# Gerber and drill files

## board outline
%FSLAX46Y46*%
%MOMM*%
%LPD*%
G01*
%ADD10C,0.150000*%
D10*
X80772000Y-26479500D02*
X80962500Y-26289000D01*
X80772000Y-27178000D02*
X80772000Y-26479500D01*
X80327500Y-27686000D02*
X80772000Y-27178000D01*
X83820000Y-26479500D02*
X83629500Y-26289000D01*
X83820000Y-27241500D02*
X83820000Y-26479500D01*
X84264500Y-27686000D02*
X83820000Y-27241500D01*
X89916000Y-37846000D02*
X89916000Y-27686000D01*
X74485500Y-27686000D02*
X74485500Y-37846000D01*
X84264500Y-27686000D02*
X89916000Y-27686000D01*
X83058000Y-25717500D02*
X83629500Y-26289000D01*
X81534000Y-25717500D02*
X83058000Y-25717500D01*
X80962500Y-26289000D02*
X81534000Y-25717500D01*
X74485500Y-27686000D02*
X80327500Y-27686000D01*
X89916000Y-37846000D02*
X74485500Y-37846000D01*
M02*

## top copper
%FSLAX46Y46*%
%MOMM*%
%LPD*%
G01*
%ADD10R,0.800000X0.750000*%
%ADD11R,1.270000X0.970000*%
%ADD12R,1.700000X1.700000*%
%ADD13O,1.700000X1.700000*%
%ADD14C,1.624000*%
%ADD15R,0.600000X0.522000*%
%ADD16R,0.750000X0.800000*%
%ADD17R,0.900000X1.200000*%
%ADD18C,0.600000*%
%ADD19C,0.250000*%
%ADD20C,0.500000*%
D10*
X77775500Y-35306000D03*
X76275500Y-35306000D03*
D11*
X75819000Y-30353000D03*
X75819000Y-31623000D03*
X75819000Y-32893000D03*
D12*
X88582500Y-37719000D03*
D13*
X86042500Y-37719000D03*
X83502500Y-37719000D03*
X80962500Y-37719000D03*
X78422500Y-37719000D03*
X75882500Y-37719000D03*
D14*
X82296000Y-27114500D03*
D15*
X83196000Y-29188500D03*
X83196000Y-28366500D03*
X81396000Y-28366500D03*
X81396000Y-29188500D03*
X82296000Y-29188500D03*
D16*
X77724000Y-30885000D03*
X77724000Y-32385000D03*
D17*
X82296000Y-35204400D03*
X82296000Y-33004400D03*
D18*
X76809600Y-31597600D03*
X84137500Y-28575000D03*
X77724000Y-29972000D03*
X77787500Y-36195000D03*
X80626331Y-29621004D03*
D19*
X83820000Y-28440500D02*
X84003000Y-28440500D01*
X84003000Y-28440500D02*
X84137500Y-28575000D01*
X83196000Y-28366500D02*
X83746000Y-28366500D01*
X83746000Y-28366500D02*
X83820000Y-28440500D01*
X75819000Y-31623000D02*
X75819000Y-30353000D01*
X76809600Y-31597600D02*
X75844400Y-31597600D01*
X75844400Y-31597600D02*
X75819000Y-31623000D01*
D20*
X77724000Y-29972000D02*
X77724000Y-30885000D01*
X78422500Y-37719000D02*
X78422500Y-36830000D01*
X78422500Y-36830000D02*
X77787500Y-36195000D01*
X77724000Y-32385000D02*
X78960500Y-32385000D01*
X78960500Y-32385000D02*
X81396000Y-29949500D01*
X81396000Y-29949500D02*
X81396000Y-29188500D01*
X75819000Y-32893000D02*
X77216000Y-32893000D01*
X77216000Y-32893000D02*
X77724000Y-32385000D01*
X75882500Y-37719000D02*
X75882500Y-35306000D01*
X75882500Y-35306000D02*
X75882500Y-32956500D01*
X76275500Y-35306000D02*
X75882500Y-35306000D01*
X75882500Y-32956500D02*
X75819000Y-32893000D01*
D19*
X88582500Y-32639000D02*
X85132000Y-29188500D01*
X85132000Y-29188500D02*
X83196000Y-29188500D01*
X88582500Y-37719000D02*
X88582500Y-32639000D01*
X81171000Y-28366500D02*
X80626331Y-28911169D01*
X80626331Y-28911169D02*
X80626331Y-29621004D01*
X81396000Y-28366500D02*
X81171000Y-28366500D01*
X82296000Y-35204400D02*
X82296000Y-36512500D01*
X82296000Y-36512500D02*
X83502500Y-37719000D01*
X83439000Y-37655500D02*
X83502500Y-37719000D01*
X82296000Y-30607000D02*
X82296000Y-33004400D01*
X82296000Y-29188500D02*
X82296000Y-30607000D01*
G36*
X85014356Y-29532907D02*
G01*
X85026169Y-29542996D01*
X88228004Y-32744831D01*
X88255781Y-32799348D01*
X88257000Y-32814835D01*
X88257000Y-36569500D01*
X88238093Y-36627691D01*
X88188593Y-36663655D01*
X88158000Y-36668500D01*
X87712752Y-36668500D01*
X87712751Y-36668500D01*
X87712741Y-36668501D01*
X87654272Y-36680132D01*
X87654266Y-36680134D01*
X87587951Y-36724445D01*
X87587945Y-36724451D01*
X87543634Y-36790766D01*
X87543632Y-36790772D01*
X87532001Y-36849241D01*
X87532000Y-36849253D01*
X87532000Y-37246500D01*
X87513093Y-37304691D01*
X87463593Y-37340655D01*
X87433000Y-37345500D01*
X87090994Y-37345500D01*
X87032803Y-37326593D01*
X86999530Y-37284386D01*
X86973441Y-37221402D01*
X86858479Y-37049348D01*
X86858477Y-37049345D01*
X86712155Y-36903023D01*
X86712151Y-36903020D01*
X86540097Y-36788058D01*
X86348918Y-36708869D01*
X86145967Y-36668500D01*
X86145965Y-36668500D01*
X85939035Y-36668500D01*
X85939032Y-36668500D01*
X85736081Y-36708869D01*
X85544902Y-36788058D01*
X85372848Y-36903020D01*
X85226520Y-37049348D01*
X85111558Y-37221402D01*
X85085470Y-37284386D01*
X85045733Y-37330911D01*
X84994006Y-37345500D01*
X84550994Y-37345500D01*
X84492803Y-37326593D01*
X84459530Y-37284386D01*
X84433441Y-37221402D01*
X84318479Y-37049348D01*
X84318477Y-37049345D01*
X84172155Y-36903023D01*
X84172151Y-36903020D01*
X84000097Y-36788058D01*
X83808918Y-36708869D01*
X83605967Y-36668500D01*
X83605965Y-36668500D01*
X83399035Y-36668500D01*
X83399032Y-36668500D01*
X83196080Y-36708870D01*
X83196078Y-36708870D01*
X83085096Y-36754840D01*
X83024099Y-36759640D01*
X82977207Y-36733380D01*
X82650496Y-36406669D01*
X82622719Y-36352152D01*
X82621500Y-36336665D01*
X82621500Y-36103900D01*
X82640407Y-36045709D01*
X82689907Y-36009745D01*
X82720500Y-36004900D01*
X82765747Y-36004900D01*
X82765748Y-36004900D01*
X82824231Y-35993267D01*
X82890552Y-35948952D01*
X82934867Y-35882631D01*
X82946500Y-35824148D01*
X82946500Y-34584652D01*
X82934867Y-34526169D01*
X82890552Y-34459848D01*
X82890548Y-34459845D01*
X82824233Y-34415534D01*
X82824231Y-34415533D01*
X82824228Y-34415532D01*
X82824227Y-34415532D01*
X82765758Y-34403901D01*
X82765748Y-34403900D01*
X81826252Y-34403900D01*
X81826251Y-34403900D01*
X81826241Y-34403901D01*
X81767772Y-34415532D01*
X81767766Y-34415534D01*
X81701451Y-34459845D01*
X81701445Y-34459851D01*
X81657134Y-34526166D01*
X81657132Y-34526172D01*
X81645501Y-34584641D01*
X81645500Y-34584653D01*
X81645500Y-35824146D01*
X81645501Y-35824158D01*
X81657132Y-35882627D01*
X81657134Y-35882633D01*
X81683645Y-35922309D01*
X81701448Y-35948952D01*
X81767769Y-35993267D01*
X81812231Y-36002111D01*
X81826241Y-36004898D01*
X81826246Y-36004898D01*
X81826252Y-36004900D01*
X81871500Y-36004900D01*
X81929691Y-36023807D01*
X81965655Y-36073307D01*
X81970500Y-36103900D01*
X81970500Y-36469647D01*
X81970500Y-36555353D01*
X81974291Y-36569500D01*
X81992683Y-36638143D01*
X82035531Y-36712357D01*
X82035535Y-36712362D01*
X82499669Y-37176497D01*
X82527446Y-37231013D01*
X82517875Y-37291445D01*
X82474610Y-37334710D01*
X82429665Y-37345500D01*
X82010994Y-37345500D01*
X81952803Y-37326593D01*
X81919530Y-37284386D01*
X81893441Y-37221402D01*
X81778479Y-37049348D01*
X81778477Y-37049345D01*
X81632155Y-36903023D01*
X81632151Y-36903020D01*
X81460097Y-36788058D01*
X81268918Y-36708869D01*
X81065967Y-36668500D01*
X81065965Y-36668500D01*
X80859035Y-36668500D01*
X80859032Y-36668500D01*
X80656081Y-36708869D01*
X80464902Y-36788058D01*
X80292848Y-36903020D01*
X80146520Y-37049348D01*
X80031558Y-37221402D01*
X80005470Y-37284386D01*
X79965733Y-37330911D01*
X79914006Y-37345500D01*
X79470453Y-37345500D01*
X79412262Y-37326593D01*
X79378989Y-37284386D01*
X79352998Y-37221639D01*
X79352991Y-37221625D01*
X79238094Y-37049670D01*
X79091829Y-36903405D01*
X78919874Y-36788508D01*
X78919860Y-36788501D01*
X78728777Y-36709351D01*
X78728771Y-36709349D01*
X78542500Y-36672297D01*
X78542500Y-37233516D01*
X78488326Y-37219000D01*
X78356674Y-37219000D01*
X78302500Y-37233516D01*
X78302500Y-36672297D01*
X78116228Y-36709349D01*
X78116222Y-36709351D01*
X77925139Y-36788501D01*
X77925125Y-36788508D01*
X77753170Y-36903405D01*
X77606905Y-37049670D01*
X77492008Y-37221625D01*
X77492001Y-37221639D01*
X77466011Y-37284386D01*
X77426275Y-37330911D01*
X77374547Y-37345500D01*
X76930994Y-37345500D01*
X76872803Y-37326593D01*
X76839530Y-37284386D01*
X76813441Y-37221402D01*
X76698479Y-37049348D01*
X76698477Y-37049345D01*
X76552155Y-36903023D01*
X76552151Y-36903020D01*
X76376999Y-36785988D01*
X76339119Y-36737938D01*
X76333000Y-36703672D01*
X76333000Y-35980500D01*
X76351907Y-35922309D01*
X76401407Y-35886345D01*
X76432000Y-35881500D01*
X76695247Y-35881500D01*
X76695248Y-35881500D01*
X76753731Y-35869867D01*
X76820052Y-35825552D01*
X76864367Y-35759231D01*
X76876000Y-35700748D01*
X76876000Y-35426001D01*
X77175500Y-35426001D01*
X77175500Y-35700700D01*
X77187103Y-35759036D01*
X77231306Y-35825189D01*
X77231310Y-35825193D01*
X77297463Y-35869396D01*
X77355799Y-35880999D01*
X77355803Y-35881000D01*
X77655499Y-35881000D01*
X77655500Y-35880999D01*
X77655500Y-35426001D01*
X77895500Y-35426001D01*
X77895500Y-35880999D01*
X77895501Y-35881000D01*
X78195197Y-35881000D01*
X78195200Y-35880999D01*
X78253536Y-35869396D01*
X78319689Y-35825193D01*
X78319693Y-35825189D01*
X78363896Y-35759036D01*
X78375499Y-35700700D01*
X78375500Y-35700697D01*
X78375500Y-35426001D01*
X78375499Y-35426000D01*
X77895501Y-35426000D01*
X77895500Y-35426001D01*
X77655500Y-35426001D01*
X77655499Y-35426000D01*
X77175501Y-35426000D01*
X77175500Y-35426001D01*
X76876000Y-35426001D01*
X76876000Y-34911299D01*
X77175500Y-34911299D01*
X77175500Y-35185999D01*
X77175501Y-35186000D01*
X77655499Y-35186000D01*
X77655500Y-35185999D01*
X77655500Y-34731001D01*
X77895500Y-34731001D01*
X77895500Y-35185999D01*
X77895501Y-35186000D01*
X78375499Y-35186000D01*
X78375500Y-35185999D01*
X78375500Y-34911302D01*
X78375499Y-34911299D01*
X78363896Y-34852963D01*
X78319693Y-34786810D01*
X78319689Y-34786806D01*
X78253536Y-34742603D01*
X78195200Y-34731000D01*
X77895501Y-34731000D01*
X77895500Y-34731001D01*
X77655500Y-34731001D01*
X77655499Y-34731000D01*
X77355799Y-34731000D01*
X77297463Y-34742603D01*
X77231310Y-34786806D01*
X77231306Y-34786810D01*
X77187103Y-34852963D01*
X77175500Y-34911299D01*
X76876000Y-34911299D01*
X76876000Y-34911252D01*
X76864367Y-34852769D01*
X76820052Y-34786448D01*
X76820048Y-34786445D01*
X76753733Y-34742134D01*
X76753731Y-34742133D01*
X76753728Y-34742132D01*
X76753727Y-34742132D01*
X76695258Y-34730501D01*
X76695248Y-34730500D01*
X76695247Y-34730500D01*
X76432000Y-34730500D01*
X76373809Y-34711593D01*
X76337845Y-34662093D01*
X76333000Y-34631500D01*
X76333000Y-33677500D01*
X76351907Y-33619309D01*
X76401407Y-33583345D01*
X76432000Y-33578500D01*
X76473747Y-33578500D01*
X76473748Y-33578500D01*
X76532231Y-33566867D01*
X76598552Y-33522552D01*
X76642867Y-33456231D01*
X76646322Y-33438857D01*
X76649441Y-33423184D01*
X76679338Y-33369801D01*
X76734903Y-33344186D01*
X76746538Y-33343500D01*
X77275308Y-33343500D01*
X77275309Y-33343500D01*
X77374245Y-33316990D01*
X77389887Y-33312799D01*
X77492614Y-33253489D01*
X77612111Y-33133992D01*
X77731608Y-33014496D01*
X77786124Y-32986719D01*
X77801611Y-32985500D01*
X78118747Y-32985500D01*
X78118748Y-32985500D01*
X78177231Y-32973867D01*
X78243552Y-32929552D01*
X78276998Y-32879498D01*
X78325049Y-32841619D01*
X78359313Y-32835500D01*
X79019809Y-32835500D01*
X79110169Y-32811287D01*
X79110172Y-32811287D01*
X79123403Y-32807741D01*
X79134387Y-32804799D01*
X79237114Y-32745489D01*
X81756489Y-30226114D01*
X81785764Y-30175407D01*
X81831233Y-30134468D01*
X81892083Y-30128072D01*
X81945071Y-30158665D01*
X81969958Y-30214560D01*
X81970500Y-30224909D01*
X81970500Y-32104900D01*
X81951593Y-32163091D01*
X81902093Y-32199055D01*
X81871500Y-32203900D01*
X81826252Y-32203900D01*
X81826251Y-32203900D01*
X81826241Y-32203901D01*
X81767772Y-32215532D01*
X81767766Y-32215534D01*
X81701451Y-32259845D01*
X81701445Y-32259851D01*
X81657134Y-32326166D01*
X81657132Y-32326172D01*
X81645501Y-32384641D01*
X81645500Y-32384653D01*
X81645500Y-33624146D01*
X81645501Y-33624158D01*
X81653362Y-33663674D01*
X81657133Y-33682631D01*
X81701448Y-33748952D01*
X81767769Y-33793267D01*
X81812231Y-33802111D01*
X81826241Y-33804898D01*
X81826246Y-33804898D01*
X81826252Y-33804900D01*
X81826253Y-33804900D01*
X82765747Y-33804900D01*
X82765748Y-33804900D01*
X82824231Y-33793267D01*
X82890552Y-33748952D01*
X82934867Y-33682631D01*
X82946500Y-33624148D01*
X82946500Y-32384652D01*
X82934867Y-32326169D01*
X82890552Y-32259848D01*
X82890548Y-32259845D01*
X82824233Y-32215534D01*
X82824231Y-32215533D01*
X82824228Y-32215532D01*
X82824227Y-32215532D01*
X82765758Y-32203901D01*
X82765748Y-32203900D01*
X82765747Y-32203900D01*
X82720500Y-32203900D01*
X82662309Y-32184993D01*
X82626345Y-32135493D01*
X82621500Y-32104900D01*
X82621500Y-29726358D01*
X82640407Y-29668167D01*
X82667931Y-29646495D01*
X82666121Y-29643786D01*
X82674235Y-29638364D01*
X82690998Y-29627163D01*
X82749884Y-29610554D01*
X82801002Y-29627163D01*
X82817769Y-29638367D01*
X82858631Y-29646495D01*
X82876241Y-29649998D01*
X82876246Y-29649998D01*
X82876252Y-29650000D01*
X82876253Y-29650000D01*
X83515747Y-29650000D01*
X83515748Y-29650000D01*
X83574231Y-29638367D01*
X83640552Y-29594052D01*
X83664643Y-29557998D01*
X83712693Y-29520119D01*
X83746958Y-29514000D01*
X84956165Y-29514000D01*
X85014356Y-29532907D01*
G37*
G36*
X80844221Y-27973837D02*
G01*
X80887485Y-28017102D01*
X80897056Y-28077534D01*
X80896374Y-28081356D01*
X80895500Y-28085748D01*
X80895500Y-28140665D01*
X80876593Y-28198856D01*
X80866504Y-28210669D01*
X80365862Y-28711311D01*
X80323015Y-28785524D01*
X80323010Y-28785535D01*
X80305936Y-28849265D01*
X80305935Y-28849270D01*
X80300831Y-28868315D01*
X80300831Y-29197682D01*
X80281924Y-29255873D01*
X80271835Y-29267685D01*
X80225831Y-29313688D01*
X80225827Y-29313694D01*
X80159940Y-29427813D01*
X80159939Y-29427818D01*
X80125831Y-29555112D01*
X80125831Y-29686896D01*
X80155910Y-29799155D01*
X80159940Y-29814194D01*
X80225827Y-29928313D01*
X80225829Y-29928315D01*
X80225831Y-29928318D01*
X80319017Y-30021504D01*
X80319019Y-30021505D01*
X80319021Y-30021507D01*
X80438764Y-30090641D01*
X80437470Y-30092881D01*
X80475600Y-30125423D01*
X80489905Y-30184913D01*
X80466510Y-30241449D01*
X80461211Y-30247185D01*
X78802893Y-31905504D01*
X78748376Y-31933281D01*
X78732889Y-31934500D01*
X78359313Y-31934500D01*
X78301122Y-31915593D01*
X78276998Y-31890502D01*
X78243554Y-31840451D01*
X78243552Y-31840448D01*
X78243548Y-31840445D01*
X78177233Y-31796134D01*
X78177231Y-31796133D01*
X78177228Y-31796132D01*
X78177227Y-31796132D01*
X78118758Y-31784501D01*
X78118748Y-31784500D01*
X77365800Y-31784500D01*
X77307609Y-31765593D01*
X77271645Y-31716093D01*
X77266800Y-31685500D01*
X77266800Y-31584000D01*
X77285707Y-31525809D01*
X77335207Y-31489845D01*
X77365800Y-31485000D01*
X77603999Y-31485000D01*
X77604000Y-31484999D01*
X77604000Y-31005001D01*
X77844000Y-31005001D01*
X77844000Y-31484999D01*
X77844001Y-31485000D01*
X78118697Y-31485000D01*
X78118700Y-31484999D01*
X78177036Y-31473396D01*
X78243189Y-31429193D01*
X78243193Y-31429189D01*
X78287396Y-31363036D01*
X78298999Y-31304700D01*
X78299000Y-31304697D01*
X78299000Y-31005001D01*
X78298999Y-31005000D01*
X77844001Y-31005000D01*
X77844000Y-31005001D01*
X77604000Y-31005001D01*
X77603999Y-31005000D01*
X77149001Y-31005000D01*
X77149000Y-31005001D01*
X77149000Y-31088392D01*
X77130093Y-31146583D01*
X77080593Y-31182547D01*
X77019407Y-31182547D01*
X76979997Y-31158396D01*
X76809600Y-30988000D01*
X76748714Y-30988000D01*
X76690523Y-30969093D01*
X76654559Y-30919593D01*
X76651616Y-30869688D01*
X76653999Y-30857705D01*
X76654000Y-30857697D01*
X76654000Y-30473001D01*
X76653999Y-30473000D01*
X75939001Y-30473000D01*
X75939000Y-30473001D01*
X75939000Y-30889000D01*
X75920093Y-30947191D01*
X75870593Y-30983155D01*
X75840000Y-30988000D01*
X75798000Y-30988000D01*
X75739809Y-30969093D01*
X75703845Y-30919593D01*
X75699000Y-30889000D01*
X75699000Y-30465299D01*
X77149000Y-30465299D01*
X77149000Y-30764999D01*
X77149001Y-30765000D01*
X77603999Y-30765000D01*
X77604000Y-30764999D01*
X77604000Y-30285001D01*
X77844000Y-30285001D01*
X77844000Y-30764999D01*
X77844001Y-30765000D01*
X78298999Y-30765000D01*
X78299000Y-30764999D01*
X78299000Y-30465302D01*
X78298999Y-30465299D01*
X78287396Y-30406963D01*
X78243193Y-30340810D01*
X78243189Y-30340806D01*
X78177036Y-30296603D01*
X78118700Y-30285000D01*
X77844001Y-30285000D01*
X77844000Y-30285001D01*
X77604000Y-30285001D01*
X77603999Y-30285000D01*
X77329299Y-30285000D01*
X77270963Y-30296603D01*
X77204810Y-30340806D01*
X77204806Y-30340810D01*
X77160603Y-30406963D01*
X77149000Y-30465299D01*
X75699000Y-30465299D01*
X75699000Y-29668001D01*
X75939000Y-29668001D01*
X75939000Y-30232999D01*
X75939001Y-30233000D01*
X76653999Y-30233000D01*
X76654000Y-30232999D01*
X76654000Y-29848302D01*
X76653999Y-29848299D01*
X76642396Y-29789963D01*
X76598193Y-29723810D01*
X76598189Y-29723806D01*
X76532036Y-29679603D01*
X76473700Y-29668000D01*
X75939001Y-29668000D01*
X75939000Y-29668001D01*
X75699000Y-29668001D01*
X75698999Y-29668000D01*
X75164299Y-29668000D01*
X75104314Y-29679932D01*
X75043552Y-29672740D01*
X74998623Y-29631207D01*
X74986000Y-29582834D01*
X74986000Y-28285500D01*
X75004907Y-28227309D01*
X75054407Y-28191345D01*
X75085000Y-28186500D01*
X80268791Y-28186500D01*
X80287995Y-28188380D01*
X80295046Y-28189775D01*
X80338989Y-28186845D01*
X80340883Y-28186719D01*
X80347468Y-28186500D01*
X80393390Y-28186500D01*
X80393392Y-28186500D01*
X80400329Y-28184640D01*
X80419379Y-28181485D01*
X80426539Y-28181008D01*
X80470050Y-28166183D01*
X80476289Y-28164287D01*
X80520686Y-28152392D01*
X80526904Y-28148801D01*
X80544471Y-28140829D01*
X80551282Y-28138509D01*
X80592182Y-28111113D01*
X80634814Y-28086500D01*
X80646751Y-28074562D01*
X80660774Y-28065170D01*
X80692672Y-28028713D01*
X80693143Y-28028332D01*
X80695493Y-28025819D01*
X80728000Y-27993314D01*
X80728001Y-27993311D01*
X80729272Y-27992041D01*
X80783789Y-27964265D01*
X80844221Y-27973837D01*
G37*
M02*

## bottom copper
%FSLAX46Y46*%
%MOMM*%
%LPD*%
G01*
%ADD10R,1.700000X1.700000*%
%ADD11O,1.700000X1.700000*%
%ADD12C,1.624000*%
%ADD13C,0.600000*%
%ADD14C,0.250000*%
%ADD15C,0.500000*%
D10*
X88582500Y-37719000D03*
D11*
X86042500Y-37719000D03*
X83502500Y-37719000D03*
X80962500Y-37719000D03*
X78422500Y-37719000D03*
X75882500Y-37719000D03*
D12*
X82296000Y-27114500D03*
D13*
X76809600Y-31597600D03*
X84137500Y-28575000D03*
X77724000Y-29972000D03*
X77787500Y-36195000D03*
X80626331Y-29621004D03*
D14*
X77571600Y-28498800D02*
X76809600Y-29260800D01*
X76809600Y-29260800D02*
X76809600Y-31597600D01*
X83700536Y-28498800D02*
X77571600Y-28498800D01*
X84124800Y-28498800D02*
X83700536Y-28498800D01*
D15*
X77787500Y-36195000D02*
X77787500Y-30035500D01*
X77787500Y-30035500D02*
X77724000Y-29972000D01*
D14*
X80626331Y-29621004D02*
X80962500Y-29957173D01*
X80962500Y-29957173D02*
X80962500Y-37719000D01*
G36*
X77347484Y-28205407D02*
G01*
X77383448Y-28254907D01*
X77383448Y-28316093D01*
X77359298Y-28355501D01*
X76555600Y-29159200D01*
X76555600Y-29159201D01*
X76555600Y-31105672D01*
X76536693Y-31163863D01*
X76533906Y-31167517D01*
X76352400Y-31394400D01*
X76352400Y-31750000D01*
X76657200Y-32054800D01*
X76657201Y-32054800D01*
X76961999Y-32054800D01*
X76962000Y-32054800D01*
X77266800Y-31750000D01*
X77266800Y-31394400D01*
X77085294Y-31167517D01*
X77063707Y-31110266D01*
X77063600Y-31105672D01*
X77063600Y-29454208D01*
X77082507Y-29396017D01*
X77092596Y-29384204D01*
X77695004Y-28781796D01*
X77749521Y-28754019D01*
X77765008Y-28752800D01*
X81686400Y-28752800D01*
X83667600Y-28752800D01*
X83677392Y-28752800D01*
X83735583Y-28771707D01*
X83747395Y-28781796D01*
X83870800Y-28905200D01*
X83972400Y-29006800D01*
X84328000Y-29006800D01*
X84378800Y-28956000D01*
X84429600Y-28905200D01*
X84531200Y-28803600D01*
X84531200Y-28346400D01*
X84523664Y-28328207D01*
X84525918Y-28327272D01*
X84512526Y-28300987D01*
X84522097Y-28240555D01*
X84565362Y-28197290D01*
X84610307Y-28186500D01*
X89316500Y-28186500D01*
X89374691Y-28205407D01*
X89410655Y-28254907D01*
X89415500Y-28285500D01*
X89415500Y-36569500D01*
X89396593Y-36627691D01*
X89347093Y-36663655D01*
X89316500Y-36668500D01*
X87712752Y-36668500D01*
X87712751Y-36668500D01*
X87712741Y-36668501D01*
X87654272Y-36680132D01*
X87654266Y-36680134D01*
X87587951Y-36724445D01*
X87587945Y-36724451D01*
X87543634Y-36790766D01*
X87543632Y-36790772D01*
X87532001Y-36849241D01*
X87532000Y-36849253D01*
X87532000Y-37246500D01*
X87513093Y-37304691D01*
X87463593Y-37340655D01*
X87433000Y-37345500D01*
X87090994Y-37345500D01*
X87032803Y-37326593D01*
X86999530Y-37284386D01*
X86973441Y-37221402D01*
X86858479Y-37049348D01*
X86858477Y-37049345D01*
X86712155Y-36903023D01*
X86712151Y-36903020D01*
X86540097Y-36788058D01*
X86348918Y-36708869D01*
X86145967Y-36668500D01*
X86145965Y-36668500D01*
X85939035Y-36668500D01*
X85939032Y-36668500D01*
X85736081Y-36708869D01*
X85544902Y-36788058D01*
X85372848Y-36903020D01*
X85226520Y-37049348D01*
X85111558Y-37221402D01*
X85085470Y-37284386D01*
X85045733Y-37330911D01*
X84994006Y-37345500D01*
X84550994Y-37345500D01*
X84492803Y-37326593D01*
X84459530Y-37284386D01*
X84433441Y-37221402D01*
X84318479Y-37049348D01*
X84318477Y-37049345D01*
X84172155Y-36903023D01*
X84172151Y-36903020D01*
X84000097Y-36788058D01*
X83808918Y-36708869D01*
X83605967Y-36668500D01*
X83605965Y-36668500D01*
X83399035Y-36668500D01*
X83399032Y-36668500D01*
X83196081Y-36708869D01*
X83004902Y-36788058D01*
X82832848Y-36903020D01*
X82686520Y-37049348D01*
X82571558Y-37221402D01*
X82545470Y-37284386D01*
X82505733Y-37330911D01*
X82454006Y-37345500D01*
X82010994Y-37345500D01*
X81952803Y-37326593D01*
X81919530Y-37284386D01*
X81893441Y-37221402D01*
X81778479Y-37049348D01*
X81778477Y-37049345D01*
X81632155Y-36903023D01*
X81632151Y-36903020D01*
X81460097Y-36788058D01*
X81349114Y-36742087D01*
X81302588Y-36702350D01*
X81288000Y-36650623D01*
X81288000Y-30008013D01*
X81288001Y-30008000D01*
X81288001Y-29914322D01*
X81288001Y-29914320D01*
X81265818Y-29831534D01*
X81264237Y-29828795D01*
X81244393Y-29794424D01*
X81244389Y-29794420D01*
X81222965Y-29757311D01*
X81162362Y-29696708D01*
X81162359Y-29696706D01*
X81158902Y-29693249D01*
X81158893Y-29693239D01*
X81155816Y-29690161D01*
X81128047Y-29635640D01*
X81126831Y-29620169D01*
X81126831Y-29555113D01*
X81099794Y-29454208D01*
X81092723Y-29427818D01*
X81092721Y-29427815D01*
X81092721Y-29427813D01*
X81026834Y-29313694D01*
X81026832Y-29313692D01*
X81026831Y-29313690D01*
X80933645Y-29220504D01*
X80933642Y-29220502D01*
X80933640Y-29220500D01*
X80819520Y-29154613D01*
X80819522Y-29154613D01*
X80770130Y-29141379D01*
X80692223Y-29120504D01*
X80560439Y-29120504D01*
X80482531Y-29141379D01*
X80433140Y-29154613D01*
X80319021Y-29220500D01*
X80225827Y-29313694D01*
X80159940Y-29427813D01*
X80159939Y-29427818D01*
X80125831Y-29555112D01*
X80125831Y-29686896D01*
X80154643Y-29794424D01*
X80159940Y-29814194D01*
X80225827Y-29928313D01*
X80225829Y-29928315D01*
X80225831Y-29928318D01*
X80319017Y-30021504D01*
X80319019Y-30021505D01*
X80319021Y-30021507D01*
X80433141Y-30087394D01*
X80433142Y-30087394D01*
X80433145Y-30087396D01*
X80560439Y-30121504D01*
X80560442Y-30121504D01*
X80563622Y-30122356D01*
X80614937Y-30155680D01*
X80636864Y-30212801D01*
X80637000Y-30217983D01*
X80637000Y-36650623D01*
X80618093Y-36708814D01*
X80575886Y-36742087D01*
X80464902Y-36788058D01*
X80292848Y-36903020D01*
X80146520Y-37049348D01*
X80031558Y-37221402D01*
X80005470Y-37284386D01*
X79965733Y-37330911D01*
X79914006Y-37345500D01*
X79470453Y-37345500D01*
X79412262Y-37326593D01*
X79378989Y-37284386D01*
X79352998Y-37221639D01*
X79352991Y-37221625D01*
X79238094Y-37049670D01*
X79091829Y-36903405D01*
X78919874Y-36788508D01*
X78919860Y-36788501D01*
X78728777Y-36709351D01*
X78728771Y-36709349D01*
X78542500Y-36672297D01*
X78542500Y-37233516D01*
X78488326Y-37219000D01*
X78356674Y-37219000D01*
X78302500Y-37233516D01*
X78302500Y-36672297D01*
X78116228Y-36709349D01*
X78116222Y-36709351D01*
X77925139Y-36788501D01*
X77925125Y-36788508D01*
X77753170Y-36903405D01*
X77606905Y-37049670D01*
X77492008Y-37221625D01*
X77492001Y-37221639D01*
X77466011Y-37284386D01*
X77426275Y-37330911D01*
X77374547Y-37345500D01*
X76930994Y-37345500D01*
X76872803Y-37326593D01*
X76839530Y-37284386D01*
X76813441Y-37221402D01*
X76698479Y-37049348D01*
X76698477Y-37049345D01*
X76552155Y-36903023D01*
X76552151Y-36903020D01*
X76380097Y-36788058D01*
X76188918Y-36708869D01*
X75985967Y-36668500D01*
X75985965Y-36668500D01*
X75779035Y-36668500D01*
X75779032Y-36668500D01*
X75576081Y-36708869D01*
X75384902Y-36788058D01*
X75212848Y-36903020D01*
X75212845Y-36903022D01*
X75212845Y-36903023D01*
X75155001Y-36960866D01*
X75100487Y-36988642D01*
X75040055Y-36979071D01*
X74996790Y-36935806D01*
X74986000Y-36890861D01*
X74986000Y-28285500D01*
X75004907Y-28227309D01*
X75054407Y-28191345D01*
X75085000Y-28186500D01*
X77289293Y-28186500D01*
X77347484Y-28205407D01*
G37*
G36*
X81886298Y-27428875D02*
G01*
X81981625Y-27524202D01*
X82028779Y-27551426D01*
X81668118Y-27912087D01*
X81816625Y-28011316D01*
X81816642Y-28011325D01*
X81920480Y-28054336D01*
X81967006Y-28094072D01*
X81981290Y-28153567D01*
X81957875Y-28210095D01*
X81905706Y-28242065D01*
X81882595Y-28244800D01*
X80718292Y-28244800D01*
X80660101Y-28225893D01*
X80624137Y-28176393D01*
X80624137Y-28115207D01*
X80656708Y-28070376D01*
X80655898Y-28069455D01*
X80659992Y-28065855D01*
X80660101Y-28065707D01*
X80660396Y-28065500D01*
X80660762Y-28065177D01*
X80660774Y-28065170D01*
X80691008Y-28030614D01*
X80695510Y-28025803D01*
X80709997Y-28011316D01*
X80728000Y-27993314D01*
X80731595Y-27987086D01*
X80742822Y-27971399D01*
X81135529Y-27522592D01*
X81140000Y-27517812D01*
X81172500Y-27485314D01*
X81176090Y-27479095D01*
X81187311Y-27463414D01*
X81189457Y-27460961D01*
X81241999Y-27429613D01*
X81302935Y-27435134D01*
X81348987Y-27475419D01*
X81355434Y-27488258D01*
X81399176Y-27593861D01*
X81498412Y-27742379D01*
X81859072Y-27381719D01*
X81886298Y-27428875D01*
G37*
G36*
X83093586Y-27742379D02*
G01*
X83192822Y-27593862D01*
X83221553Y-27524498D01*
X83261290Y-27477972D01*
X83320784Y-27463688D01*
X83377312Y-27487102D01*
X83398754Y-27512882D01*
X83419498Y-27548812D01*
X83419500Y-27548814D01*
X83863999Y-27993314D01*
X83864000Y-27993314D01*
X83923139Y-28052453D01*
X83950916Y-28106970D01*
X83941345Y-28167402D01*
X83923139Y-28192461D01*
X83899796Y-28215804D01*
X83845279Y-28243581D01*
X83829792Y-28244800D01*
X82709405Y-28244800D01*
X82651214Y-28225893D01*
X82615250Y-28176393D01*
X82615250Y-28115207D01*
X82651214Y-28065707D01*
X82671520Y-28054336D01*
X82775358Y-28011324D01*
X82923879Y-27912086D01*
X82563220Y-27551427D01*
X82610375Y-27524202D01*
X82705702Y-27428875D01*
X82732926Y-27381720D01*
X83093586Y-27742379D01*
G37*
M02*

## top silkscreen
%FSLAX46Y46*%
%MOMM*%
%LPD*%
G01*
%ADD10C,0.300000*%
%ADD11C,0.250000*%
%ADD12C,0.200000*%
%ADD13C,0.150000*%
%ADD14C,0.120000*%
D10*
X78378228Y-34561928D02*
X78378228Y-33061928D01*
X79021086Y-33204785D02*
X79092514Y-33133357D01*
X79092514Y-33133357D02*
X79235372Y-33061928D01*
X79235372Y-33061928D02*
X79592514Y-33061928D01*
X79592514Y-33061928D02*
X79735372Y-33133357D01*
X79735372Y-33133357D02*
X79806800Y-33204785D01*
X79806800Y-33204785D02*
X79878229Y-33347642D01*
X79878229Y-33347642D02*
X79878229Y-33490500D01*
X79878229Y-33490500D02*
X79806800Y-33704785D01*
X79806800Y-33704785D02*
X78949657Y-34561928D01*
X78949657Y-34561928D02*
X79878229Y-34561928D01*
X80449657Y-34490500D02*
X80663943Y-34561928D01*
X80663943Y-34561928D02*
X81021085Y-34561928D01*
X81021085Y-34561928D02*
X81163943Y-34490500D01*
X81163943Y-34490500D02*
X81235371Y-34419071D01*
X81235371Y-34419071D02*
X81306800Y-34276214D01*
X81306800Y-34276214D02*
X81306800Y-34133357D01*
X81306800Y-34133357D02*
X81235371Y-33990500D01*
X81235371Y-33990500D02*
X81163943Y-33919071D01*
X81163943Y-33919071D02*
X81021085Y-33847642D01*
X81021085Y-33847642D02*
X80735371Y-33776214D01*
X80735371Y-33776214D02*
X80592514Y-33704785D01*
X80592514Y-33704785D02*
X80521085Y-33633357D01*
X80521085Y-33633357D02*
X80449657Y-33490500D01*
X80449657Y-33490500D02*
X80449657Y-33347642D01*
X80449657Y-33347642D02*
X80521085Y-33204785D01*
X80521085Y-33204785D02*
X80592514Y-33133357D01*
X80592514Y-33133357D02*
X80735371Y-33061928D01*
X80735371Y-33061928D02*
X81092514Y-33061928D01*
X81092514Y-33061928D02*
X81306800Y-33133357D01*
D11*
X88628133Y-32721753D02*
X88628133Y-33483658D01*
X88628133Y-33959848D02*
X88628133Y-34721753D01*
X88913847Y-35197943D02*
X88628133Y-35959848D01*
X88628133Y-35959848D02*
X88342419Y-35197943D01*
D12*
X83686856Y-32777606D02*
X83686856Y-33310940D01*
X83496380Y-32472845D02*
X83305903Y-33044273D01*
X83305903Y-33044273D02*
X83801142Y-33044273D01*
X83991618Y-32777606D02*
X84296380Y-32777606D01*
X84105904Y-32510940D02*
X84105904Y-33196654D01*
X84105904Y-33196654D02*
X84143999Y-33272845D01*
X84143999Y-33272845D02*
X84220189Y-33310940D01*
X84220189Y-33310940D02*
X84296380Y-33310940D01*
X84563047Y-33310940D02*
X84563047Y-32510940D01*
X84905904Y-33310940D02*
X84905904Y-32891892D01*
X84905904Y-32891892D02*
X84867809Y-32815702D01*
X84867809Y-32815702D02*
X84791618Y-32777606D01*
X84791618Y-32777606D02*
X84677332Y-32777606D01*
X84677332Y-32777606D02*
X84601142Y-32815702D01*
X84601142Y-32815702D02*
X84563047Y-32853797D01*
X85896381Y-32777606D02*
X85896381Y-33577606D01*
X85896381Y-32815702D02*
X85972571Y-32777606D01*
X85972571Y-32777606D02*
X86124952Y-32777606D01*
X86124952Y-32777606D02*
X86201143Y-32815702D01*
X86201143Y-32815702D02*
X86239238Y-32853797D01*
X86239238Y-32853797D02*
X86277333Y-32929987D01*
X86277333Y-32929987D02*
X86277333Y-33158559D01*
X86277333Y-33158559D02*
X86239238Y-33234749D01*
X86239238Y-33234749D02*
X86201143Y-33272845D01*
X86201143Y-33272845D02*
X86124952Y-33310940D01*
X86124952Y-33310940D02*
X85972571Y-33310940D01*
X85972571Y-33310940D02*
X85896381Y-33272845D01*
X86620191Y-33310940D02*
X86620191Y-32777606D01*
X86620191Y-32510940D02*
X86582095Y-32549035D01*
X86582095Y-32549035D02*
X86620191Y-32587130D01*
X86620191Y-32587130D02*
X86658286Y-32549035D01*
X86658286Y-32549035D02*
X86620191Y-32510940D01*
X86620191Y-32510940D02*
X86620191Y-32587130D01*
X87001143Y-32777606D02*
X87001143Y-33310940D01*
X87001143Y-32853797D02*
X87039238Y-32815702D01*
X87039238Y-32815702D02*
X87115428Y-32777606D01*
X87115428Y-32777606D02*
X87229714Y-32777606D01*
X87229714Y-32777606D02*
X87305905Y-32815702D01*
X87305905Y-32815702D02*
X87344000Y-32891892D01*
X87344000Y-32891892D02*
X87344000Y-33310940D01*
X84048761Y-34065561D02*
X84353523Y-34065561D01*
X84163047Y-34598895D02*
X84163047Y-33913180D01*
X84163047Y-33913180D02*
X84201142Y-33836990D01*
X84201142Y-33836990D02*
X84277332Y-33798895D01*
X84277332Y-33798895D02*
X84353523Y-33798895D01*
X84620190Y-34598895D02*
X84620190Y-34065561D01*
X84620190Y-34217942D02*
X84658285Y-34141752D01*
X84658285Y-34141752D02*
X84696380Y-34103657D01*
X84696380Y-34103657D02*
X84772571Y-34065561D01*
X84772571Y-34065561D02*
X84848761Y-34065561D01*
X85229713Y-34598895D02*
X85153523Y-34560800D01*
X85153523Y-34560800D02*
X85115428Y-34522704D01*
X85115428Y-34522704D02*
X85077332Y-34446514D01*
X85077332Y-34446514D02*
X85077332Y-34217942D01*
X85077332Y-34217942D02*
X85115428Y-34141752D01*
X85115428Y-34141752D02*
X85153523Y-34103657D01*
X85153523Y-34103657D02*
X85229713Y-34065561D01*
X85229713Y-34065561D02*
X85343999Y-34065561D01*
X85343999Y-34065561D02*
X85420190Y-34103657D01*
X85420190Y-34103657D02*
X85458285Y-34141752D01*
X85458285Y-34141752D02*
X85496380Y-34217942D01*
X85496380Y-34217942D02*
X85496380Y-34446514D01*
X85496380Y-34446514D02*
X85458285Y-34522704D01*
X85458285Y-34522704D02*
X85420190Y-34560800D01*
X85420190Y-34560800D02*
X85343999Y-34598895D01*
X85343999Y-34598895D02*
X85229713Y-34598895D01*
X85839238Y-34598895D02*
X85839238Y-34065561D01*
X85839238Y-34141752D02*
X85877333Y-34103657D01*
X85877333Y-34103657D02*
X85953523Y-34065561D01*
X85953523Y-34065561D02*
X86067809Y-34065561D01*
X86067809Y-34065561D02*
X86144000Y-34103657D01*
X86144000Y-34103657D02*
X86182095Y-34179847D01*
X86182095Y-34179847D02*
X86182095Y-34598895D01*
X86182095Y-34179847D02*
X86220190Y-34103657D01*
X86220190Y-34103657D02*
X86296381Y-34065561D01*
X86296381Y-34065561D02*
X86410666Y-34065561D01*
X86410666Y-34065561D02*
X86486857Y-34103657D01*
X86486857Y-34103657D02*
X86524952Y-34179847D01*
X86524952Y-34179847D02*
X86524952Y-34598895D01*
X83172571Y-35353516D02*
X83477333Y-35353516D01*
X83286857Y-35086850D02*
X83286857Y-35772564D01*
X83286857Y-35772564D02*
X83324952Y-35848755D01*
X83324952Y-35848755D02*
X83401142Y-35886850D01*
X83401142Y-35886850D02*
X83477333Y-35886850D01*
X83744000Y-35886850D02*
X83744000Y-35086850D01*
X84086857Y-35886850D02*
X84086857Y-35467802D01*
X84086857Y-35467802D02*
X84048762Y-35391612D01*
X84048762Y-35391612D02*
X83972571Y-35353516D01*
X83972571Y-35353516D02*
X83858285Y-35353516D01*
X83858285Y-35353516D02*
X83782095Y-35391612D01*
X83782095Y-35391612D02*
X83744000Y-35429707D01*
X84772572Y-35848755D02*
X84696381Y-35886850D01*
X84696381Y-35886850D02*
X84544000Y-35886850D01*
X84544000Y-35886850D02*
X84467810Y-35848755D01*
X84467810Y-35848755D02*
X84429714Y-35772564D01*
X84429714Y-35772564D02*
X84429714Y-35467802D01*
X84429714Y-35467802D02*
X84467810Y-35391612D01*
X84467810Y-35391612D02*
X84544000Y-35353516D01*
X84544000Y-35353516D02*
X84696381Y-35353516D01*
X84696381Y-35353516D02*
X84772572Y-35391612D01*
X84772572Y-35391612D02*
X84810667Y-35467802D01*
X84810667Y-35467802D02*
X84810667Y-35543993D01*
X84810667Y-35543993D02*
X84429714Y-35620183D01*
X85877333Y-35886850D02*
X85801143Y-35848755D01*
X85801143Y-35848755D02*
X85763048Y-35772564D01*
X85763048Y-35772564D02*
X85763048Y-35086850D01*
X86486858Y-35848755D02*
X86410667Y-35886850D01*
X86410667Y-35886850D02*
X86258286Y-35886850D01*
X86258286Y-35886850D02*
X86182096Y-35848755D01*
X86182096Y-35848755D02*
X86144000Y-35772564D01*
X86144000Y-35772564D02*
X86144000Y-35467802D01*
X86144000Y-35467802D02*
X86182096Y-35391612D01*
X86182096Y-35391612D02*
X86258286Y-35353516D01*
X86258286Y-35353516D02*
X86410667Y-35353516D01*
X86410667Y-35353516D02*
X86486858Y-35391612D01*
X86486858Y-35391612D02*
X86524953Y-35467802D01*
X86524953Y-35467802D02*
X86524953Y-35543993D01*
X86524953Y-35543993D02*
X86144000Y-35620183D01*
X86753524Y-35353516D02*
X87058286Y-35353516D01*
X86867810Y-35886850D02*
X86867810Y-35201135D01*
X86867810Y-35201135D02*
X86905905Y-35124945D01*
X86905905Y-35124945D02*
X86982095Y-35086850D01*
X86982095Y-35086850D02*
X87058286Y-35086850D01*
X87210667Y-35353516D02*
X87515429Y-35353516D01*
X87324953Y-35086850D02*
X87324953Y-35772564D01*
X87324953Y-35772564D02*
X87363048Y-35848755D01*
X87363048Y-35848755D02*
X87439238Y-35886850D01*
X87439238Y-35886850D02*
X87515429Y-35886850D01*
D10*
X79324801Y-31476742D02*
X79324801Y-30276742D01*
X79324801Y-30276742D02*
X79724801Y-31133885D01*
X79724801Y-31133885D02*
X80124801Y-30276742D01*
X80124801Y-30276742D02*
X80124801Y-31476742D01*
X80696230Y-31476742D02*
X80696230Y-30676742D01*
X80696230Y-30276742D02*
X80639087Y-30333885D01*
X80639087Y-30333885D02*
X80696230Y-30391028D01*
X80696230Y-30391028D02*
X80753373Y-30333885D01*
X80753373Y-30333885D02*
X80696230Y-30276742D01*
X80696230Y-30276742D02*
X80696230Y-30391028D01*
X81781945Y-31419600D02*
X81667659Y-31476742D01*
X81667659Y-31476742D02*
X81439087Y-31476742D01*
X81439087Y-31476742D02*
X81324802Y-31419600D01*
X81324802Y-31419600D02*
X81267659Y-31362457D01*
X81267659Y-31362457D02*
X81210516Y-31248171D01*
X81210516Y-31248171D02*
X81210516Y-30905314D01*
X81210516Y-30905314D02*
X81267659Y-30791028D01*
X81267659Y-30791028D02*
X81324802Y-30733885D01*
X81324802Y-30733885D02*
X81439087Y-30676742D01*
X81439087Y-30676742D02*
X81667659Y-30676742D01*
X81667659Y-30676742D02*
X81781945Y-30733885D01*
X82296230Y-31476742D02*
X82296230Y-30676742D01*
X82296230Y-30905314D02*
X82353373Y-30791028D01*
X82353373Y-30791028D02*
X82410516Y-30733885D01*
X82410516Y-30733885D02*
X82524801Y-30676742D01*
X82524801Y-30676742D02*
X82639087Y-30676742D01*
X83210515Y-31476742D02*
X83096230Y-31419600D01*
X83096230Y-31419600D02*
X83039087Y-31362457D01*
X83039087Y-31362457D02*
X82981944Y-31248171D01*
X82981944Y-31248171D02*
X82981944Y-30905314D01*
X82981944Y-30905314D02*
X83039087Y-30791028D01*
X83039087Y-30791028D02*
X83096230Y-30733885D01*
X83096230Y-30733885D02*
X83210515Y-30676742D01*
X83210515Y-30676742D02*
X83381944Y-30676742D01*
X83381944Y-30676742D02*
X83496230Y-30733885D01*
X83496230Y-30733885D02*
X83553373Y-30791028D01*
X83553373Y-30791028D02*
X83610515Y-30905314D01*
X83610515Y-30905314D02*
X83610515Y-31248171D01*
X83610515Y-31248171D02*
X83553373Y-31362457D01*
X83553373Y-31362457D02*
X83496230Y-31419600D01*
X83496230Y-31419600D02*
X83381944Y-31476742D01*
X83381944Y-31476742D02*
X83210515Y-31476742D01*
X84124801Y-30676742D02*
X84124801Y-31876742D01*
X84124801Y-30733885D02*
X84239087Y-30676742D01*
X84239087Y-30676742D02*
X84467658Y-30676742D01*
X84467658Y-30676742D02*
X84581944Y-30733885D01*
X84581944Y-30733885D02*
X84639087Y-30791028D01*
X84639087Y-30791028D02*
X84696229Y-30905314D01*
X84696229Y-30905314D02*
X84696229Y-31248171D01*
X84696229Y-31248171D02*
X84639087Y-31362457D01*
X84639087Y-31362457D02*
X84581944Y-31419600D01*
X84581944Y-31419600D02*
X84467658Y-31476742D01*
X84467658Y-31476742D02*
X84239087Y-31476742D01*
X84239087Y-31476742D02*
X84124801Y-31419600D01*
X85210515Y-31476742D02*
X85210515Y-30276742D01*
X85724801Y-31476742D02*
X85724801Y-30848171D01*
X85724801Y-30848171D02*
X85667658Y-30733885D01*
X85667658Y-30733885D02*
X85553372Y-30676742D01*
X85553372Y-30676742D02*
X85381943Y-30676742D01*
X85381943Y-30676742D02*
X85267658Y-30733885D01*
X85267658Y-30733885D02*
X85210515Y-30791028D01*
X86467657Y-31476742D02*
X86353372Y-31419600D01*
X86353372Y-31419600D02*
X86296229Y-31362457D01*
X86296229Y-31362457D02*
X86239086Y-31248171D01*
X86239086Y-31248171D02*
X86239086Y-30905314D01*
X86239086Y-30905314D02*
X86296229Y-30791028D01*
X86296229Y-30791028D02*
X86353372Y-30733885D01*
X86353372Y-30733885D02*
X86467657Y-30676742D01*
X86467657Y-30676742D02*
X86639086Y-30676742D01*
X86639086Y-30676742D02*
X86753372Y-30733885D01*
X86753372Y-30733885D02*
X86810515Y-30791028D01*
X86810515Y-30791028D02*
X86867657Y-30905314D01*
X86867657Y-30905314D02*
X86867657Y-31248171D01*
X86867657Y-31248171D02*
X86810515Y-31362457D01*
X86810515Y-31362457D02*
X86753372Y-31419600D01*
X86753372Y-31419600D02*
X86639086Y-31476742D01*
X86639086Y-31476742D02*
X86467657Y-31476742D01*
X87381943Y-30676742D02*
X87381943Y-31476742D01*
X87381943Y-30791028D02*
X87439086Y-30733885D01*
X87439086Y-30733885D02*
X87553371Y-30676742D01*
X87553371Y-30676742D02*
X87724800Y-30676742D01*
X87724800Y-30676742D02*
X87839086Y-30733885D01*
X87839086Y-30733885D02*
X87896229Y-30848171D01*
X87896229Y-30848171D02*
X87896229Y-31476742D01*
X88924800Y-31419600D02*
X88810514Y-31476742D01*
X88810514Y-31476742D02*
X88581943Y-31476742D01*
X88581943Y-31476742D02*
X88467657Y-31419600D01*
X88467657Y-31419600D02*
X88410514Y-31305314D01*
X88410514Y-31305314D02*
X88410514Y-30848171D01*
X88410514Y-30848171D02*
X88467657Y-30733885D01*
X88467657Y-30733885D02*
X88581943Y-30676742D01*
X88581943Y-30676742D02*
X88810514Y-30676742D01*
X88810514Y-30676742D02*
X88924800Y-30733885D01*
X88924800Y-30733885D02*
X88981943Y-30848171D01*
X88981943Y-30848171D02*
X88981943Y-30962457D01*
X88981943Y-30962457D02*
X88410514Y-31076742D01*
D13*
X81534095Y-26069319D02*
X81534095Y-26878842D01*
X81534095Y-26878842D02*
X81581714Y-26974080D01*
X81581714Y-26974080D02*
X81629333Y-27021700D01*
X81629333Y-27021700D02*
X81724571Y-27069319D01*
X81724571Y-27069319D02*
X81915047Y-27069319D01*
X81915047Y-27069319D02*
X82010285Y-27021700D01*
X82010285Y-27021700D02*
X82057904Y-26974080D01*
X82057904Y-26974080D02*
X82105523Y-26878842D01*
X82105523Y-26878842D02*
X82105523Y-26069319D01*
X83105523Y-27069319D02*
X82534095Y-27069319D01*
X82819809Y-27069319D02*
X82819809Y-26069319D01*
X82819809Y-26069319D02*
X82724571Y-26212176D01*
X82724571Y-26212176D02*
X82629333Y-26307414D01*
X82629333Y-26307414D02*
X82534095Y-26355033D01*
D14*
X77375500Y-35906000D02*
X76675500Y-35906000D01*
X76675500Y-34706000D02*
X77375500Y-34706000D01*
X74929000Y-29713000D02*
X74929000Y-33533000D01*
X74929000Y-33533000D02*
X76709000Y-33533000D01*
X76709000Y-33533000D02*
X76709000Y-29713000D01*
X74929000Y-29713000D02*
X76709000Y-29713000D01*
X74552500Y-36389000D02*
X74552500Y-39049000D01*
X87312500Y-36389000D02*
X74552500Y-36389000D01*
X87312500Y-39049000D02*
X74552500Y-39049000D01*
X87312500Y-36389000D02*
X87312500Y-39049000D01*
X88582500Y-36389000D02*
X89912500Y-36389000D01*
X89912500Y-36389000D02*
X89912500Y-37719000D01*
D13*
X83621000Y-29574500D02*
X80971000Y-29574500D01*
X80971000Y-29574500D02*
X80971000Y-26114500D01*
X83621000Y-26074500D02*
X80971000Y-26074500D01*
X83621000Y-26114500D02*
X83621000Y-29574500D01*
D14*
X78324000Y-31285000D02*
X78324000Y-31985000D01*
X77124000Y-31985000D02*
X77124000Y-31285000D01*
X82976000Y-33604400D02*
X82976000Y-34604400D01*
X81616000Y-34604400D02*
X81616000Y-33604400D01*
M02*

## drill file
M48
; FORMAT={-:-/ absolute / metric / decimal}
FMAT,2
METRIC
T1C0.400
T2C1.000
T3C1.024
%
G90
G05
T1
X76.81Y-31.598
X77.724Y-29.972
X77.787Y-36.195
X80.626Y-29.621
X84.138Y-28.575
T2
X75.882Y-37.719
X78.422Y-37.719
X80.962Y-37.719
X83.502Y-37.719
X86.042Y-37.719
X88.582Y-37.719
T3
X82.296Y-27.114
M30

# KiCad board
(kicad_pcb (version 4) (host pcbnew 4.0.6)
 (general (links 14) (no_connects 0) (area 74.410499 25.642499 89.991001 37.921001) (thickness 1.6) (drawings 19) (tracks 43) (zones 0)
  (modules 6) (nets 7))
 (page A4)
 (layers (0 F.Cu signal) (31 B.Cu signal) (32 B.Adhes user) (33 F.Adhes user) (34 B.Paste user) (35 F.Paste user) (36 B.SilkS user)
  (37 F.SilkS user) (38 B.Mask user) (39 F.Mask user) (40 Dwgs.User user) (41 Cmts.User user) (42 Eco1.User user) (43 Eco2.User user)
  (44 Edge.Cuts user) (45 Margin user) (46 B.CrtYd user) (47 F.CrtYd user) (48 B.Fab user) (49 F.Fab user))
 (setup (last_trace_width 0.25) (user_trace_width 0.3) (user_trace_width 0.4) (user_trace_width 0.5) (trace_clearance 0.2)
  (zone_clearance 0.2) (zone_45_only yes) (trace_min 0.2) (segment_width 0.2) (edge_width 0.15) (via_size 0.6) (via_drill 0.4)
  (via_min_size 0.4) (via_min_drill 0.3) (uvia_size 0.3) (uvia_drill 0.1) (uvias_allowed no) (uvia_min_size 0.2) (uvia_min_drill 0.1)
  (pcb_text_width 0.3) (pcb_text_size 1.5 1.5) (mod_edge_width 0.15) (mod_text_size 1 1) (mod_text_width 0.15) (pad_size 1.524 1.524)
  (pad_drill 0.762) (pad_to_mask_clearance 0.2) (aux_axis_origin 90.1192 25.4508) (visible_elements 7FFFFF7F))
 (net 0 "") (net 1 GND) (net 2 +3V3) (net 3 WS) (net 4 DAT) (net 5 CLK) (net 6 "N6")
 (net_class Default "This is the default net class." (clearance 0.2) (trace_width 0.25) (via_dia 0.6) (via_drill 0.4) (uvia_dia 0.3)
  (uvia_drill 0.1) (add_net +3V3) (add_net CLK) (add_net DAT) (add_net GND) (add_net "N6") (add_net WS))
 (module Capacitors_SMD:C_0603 (layer F.Cu) (at 77.0255 35.306)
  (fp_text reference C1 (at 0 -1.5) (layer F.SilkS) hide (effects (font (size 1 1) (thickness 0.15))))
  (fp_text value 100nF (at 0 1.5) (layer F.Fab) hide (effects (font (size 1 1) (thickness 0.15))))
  (fp_line (start 0.35 0.6) (end -0.35 0.6) (layer F.SilkS) (width 0.12))
  (fp_line (start -0.35 -0.6) (end 0.35 -0.6) (layer F.SilkS) (width 0.12))
  (pad 2 smd rect (at 0.75 0) (size 0.8 0.75) (layers F.Cu F.Paste F.Mask) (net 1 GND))
  (pad 1 smd rect (at -0.75 0) (size 0.8 0.75) (layers F.Cu F.Paste F.Mask) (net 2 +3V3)))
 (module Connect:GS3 (layer F.Cu) (at 75.819 31.623)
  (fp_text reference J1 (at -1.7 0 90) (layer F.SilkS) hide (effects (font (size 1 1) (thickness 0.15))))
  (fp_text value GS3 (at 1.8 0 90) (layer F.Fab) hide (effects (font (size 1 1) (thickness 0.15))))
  (fp_line (start -0.89 -1.91) (end -0.89 1.91) (layer F.SilkS) (width 0.12))
  (fp_line (start -0.89 1.91) (end 0.89 1.91) (layer F.SilkS) (width 0.12))
  (fp_line (start 0.89 1.91) (end 0.89 -1.91) (layer F.SilkS) (width 0.12))
  (fp_line (start -0.89 -1.91) (end 0.89 -1.91) (layer F.SilkS) (width 0.12))
  (pad 1 smd rect (at 0 -1.27) (size 1.27 0.97) (layers F.Cu F.Paste F.Mask) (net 1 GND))
  (pad 2 smd rect (at 0 0) (size 1.27 0.97) (layers F.Cu F.Paste F.Mask) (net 1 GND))
  (pad 3 smd rect (at 0 1.27) (size 1.27 0.97) (layers F.Cu F.Paste F.Mask) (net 2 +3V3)))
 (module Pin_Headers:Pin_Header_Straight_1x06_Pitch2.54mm (layer F.Cu) (at 88.5825 37.719 270)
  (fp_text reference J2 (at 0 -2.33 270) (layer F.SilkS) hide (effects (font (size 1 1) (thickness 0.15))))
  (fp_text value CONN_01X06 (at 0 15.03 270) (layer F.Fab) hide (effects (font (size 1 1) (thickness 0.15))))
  (fp_line (start -1.33 14.03) (end 1.33 14.03) (layer F.SilkS) (width 0.12))
  (fp_line (start -1.33 1.27) (end -1.33 14.03) (layer F.SilkS) (width 0.12))
  (fp_line (start 1.33 1.27) (end 1.33 14.03) (layer F.SilkS) (width 0.12))
  (fp_line (start -1.33 1.27) (end 1.33 1.27) (layer F.SilkS) (width 0.12))
  (fp_line (start -1.33 0) (end -1.33 -1.33) (layer F.SilkS) (width 0.12))
  (fp_line (start -1.33 -1.33) (end 0 -1.33) (layer F.SilkS) (width 0.12))
  (pad 1 thru_hole rect (at 0 0 270) (size 1.7 1.7) (drill 1) (layers *.Cu *.Mask) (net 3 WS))
  (pad 2 thru_hole oval (at 0 2.54 270) (size 1.7 1.7) (drill 1) (layers *.Cu *.Mask))
  (pad 3 thru_hole oval (at 0 5.08 270) (size 1.7 1.7) (drill 1) (layers *.Cu *.Mask) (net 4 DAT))
  (pad 4 thru_hole oval (at 0 7.62 270) (size 1.7 1.7) (drill 1) (layers *.Cu *.Mask) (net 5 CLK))
  (pad 5 thru_hole oval (at 0 10.16 270) (size 1.7 1.7) (drill 1) (layers *.Cu *.Mask) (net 1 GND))
  (pad 6 thru_hole oval (at 0 12.7 270) (size 1.7 1.7) (drill 1) (layers *.Cu *.Mask) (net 2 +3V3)))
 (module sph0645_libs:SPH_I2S (layer F.Cu) (at 82.296 27.1145 180)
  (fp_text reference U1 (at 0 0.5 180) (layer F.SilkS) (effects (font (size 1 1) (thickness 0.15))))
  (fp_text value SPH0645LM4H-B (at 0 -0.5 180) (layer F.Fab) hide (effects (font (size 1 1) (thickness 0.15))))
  (fp_line (start -1.325 -2.46) (end 1.325 -2.46) (layer F.SilkS) (width 0.15))
  (fp_line (start 1.325 -2.46) (end 1.325 1) (layer F.SilkS) (width 0.15))
  (fp_line (start -1.325 1.04) (end 1.325 1.04) (layer F.SilkS) (width 0.15))
  (fp_line (start -1.325 1) (end -1.325 -2.46) (layer F.SilkS) (width 0.15))
  (pad 3 thru_hole circle (at 0 0 180) (size 1.624 1.624) (drill 1.024) (layers *.Cu *.Mask) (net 1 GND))
  (pad 1 smd rect (at -0.9 -2.074 180) (size 0.6 0.522) (layers F.Cu F.Paste F.Mask) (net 3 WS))
  (pad 2 smd rect (at -0.9 -1.252 180) (size 0.6 0.522) (layers F.Cu F.Paste F.Mask) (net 1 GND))
  (pad 4 smd rect (at 0.9 -1.252 180) (size 0.6 0.522) (layers F.Cu F.Paste F.Mask) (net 5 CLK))
  (pad 5 smd rect (at 0.9 -2.074 180) (size 0.6 0.522) (layers F.Cu F.Paste F.Mask) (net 2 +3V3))
  (pad 6 smd rect (at 0 -2.074 180) (size 0.6 0.522) (layers F.Cu F.Paste F.Mask) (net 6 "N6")))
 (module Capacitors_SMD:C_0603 (layer F.Cu) (at 77.724 31.635 90)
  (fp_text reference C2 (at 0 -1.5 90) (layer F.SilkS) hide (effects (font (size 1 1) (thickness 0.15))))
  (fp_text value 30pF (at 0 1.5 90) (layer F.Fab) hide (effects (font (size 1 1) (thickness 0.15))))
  (fp_line (start 0.35 0.6) (end -0.35 0.6) (layer F.SilkS) (width 0.12))
  (fp_line (start -0.35 -0.6) (end 0.35 -0.6) (layer F.SilkS) (width 0.12))
  (pad 2 smd rect (at 0.75 0 90) (size 0.8 0.75) (layers F.Cu F.Paste F.Mask) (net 1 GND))
  (pad 1 smd rect (at -0.75 0 90) (size 0.8 0.75) (layers F.Cu F.Paste F.Mask) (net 2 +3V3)))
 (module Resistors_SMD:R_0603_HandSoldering (layer F.Cu) (at 82.296 34.1044 90)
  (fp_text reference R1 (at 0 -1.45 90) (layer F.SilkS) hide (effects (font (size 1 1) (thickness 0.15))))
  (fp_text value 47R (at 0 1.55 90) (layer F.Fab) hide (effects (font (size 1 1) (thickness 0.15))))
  (fp_line (start 0.5 0.68) (end -0.5 0.68) (layer F.SilkS) (width 0.12))
  (fp_line (start -0.5 -0.68) (end 0.5 -0.68) (layer F.SilkS) (width 0.12))
  (pad 1 smd rect (at -1.1 0 90) (size 1.2 0.9) (layers F.Cu F.Paste F.Mask) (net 4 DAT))
  (pad 2 smd rect (at 1.1 0 90) (size 1.2 0.9) (layers F.Cu F.Paste F.Mask) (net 6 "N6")))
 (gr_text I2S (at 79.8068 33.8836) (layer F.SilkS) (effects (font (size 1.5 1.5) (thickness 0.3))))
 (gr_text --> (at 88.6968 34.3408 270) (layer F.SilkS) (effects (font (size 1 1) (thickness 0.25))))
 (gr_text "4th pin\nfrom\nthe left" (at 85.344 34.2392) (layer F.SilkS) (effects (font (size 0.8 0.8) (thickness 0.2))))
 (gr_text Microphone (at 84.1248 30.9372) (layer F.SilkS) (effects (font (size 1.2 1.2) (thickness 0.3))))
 (gr_line (start 80.772 26.4795) (end 80.9625 26.289) (layer Edge.Cuts) (width 0.15))
 (gr_line (start 80.772 27.178) (end 80.772 26.4795) (layer Edge.Cuts) (width 0.15))
 (gr_line (start 80.3275 27.686) (end 80.772 27.178) (layer Edge.Cuts) (width 0.15))
 (gr_line (start 83.82 26.4795) (end 83.6295 26.289) (layer Edge.Cuts) (width 0.15))
 (gr_line (start 83.82 27.2415) (end 83.82 26.4795) (layer Edge.Cuts) (width 0.15))
 (gr_line (start 84.2645 27.686) (end 83.82 27.2415) (layer Edge.Cuts) (width 0.15))
 (gr_line (start 89.916 37.846) (end 89.916 27.686) (layer Edge.Cuts) (width 0.15))
 (gr_line (start 74.4855 27.686) (end 74.4855 37.846) (layer Edge.Cuts) (width 0.15))
 (gr_line (start 84.2645 27.686) (end 89.916 27.686) (layer Edge.Cuts) (width 0.15))
 (gr_line (start 83.058 25.7175) (end 83.6295 26.289) (layer Edge.Cuts) (width 0.15))
 (gr_line (start 81.534 25.7175) (end 83.058 25.7175) (layer Edge.Cuts) (width 0.15))
 (gr_line (start 80.9625 26.289) (end 81.534 25.7175) (layer Edge.Cuts) (width 0.15))
 (gr_line (start 74.4855 27.686) (end 80.3275 27.686) (layer Edge.Cuts) (width 0.15))
 (gr_line (start 89.916 37.846) (end 74.4855 37.846) (layer Edge.Cuts) (width 0.15))
 (segment (start 83.82 28.4405) (end 84.003 28.4405) (width 0.25) (layer F.Cu) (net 1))
 (segment (start 84.003 28.4405) (end 84.1375 28.575) (width 0.25) (layer F.Cu) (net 1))
 (segment (start 83.196 28.3665) (end 83.746 28.3665) (width 0.25) (layer F.Cu) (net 1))
 (segment (start 83.746 28.3665) (end 83.82 28.4405) (width 0.25) (layer F.Cu) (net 1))
 (segment (start 75.819 31.623) (end 75.819 30.353) (width 0.25) (layer F.Cu) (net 1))
 (segment (start 76.8096 31.5976) (end 75.8444 31.5976) (width 0.25) (layer F.Cu) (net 1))
 (segment (start 75.8444 31.5976) (end 75.819 31.623) (width 0.25) (layer F.Cu) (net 1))
 (segment (start 77.5716 28.4988) (end 76.8096 29.2608) (width 0.25) (layer B.Cu) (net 1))
 (segment (start 76.8096 29.2608) (end 76.8096 31.5976) (width 0.25) (layer B.Cu) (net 1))
 (via (at 76.8096 31.5976) (size 0.6) (drill 0.4) (layers F.Cu B.Cu) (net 1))
 (segment (start 83.700536 28.4988) (end 77.5716 28.4988) (width 0.25) (layer B.Cu) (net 1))
 (segment (start 84.1248 28.4988) (end 83.700536 28.4988) (width 0.25) (layer B.Cu) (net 1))
 (via (at 84.1375 28.575) (size 0.6) (drill 0.4) (layers F.Cu B.Cu) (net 1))
 (segment (start 77.724 29.972) (end 77.724 30.885) (width 0.5) (layer F.Cu) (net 1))
 (segment (start 77.7875 36.195) (end 77.7875 30.0355) (width 0.5) (layer B.Cu) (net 1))
 (segment (start 77.7875 30.0355) (end 77.724 29.972) (width 0.5) (layer B.Cu) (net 1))
 (via (at 77.724 29.972) (size 0.6) (drill 0.4) (layers F.Cu B.Cu) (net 1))
 (segment (start 78.4225 37.719) (end 78.4225 36.83) (width 0.5) (layer F.Cu) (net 1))
 (segment (start 78.4225 36.83) (end 77.7875 36.195) (width 0.5) (layer F.Cu) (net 1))
 (via (at 77.7875 36.195) (size 0.6) (drill 0.4) (layers F.Cu B.Cu) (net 1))
 (segment (start 77.724 32.385) (end 78.9605 32.385) (width 0.5) (layer F.Cu) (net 2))
 (segment (start 78.9605 32.385) (end 81.396 29.9495) (width 0.5) (layer F.Cu) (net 2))
 (segment (start 81.396 29.9495) (end 81.396 29.1885) (width 0.5) (layer F.Cu) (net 2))
 (segment (start 75.819 32.893) (end 77.216 32.893) (width 0.5) (layer F.Cu) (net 2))
 (segment (start 77.216 32.893) (end 77.724 32.385) (width 0.5) (layer F.Cu) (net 2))
 (segment (start 75.8825 37.719) (end 75.8825 35.306) (width 0.5) (layer F.Cu) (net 2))
 (segment (start 75.8825 35.306) (end 75.8825 32.9565) (width 0.5) (layer F.Cu) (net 2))
 (segment (start 76.2755 35.306) (end 75.8825 35.306) (width 0.5) (layer F.Cu) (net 2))
 (segment (start 75.8825 32.9565) (end 75.819 32.893) (width 0.5) (layer F.Cu) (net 2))
 (segment (start 88.5825 32.639) (end 85.132 29.1885) (width 0.25) (layer F.Cu) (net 3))
 (segment (start 85.132 29.1885) (end 83.196 29.1885) (width 0.25) (layer F.Cu) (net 3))
 (segment (start 88.5825 37.719) (end 88.5825 32.639) (width 0.25) (layer F.Cu) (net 3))
 (segment (start 80.626331 29.621004) (end 80.9625 29.957173) (width 0.25) (layer B.Cu) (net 5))
 (segment (start 80.9625 29.957173) (end 80.9625 37.719) (width 0.25) (layer B.Cu) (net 5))
 (segment (start 81.171 28.3665) (end 80.626331 28.911169) (width 0.25) (layer F.Cu) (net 5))
 (segment (start 80.626331 28.911169) (end 80.626331 29.621004) (width 0.25) (layer F.Cu) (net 5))
 (via (at 80.626331 29.621004) (size 0.6) (drill 0.4) (layers F.Cu B.Cu) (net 5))
 (segment (start 81.396 28.3665) (end 81.171 28.3665) (width 0.25) (layer F.Cu) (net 5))
 (segment (start 82.296 35.2044) (end 82.296 36.5125) (width 0.25) (layer F.Cu) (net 4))
 (segment (start 82.296 36.5125) (end 83.5025 37.719) (width 0.25) (layer F.Cu) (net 4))
 (segment (start 83.439 37.6555) (end 83.5025 37.719) (width 0.25) (layer F.Cu) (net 4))
 (segment (start 82.296 30.607) (end 82.296 33.0044) (width 0.25) (layer F.Cu) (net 6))
 (segment (start 82.296 29.1885) (end 82.296 30.607) (width 0.25) (layer F.Cu) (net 6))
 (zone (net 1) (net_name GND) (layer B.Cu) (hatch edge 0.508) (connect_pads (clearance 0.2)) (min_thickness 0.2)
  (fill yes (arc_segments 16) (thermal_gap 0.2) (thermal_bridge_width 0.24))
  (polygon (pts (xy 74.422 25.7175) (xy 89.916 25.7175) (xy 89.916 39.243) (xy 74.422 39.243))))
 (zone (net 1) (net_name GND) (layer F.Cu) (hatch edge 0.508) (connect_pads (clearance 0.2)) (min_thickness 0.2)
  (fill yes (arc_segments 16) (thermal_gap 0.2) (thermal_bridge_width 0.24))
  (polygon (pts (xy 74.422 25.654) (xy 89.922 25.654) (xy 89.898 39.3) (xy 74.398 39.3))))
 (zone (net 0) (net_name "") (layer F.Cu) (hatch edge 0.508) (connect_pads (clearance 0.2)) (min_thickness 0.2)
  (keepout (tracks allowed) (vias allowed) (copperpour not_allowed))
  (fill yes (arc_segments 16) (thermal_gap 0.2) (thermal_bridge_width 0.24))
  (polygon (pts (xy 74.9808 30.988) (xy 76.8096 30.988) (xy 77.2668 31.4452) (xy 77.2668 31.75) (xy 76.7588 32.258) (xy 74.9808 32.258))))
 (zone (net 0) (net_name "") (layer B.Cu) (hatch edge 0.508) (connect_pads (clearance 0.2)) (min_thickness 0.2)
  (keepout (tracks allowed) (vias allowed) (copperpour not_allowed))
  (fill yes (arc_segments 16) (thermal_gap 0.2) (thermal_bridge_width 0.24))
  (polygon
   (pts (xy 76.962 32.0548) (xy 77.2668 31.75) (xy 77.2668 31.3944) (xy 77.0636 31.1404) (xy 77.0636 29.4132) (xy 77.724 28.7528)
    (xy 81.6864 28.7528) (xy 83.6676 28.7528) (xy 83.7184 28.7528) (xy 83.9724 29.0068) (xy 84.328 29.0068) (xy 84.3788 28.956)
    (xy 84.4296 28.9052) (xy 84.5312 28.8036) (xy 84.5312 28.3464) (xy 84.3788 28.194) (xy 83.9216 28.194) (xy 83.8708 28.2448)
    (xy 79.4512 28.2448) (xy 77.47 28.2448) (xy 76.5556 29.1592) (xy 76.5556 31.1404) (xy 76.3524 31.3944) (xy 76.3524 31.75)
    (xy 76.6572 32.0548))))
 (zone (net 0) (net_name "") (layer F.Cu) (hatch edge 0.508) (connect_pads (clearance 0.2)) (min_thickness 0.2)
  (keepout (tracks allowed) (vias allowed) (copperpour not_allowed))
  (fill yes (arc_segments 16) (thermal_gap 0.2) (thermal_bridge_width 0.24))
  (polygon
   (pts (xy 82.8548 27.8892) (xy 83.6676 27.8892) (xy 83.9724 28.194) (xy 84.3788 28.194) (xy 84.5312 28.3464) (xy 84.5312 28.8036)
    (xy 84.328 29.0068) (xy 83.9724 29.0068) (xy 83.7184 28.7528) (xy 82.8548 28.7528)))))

